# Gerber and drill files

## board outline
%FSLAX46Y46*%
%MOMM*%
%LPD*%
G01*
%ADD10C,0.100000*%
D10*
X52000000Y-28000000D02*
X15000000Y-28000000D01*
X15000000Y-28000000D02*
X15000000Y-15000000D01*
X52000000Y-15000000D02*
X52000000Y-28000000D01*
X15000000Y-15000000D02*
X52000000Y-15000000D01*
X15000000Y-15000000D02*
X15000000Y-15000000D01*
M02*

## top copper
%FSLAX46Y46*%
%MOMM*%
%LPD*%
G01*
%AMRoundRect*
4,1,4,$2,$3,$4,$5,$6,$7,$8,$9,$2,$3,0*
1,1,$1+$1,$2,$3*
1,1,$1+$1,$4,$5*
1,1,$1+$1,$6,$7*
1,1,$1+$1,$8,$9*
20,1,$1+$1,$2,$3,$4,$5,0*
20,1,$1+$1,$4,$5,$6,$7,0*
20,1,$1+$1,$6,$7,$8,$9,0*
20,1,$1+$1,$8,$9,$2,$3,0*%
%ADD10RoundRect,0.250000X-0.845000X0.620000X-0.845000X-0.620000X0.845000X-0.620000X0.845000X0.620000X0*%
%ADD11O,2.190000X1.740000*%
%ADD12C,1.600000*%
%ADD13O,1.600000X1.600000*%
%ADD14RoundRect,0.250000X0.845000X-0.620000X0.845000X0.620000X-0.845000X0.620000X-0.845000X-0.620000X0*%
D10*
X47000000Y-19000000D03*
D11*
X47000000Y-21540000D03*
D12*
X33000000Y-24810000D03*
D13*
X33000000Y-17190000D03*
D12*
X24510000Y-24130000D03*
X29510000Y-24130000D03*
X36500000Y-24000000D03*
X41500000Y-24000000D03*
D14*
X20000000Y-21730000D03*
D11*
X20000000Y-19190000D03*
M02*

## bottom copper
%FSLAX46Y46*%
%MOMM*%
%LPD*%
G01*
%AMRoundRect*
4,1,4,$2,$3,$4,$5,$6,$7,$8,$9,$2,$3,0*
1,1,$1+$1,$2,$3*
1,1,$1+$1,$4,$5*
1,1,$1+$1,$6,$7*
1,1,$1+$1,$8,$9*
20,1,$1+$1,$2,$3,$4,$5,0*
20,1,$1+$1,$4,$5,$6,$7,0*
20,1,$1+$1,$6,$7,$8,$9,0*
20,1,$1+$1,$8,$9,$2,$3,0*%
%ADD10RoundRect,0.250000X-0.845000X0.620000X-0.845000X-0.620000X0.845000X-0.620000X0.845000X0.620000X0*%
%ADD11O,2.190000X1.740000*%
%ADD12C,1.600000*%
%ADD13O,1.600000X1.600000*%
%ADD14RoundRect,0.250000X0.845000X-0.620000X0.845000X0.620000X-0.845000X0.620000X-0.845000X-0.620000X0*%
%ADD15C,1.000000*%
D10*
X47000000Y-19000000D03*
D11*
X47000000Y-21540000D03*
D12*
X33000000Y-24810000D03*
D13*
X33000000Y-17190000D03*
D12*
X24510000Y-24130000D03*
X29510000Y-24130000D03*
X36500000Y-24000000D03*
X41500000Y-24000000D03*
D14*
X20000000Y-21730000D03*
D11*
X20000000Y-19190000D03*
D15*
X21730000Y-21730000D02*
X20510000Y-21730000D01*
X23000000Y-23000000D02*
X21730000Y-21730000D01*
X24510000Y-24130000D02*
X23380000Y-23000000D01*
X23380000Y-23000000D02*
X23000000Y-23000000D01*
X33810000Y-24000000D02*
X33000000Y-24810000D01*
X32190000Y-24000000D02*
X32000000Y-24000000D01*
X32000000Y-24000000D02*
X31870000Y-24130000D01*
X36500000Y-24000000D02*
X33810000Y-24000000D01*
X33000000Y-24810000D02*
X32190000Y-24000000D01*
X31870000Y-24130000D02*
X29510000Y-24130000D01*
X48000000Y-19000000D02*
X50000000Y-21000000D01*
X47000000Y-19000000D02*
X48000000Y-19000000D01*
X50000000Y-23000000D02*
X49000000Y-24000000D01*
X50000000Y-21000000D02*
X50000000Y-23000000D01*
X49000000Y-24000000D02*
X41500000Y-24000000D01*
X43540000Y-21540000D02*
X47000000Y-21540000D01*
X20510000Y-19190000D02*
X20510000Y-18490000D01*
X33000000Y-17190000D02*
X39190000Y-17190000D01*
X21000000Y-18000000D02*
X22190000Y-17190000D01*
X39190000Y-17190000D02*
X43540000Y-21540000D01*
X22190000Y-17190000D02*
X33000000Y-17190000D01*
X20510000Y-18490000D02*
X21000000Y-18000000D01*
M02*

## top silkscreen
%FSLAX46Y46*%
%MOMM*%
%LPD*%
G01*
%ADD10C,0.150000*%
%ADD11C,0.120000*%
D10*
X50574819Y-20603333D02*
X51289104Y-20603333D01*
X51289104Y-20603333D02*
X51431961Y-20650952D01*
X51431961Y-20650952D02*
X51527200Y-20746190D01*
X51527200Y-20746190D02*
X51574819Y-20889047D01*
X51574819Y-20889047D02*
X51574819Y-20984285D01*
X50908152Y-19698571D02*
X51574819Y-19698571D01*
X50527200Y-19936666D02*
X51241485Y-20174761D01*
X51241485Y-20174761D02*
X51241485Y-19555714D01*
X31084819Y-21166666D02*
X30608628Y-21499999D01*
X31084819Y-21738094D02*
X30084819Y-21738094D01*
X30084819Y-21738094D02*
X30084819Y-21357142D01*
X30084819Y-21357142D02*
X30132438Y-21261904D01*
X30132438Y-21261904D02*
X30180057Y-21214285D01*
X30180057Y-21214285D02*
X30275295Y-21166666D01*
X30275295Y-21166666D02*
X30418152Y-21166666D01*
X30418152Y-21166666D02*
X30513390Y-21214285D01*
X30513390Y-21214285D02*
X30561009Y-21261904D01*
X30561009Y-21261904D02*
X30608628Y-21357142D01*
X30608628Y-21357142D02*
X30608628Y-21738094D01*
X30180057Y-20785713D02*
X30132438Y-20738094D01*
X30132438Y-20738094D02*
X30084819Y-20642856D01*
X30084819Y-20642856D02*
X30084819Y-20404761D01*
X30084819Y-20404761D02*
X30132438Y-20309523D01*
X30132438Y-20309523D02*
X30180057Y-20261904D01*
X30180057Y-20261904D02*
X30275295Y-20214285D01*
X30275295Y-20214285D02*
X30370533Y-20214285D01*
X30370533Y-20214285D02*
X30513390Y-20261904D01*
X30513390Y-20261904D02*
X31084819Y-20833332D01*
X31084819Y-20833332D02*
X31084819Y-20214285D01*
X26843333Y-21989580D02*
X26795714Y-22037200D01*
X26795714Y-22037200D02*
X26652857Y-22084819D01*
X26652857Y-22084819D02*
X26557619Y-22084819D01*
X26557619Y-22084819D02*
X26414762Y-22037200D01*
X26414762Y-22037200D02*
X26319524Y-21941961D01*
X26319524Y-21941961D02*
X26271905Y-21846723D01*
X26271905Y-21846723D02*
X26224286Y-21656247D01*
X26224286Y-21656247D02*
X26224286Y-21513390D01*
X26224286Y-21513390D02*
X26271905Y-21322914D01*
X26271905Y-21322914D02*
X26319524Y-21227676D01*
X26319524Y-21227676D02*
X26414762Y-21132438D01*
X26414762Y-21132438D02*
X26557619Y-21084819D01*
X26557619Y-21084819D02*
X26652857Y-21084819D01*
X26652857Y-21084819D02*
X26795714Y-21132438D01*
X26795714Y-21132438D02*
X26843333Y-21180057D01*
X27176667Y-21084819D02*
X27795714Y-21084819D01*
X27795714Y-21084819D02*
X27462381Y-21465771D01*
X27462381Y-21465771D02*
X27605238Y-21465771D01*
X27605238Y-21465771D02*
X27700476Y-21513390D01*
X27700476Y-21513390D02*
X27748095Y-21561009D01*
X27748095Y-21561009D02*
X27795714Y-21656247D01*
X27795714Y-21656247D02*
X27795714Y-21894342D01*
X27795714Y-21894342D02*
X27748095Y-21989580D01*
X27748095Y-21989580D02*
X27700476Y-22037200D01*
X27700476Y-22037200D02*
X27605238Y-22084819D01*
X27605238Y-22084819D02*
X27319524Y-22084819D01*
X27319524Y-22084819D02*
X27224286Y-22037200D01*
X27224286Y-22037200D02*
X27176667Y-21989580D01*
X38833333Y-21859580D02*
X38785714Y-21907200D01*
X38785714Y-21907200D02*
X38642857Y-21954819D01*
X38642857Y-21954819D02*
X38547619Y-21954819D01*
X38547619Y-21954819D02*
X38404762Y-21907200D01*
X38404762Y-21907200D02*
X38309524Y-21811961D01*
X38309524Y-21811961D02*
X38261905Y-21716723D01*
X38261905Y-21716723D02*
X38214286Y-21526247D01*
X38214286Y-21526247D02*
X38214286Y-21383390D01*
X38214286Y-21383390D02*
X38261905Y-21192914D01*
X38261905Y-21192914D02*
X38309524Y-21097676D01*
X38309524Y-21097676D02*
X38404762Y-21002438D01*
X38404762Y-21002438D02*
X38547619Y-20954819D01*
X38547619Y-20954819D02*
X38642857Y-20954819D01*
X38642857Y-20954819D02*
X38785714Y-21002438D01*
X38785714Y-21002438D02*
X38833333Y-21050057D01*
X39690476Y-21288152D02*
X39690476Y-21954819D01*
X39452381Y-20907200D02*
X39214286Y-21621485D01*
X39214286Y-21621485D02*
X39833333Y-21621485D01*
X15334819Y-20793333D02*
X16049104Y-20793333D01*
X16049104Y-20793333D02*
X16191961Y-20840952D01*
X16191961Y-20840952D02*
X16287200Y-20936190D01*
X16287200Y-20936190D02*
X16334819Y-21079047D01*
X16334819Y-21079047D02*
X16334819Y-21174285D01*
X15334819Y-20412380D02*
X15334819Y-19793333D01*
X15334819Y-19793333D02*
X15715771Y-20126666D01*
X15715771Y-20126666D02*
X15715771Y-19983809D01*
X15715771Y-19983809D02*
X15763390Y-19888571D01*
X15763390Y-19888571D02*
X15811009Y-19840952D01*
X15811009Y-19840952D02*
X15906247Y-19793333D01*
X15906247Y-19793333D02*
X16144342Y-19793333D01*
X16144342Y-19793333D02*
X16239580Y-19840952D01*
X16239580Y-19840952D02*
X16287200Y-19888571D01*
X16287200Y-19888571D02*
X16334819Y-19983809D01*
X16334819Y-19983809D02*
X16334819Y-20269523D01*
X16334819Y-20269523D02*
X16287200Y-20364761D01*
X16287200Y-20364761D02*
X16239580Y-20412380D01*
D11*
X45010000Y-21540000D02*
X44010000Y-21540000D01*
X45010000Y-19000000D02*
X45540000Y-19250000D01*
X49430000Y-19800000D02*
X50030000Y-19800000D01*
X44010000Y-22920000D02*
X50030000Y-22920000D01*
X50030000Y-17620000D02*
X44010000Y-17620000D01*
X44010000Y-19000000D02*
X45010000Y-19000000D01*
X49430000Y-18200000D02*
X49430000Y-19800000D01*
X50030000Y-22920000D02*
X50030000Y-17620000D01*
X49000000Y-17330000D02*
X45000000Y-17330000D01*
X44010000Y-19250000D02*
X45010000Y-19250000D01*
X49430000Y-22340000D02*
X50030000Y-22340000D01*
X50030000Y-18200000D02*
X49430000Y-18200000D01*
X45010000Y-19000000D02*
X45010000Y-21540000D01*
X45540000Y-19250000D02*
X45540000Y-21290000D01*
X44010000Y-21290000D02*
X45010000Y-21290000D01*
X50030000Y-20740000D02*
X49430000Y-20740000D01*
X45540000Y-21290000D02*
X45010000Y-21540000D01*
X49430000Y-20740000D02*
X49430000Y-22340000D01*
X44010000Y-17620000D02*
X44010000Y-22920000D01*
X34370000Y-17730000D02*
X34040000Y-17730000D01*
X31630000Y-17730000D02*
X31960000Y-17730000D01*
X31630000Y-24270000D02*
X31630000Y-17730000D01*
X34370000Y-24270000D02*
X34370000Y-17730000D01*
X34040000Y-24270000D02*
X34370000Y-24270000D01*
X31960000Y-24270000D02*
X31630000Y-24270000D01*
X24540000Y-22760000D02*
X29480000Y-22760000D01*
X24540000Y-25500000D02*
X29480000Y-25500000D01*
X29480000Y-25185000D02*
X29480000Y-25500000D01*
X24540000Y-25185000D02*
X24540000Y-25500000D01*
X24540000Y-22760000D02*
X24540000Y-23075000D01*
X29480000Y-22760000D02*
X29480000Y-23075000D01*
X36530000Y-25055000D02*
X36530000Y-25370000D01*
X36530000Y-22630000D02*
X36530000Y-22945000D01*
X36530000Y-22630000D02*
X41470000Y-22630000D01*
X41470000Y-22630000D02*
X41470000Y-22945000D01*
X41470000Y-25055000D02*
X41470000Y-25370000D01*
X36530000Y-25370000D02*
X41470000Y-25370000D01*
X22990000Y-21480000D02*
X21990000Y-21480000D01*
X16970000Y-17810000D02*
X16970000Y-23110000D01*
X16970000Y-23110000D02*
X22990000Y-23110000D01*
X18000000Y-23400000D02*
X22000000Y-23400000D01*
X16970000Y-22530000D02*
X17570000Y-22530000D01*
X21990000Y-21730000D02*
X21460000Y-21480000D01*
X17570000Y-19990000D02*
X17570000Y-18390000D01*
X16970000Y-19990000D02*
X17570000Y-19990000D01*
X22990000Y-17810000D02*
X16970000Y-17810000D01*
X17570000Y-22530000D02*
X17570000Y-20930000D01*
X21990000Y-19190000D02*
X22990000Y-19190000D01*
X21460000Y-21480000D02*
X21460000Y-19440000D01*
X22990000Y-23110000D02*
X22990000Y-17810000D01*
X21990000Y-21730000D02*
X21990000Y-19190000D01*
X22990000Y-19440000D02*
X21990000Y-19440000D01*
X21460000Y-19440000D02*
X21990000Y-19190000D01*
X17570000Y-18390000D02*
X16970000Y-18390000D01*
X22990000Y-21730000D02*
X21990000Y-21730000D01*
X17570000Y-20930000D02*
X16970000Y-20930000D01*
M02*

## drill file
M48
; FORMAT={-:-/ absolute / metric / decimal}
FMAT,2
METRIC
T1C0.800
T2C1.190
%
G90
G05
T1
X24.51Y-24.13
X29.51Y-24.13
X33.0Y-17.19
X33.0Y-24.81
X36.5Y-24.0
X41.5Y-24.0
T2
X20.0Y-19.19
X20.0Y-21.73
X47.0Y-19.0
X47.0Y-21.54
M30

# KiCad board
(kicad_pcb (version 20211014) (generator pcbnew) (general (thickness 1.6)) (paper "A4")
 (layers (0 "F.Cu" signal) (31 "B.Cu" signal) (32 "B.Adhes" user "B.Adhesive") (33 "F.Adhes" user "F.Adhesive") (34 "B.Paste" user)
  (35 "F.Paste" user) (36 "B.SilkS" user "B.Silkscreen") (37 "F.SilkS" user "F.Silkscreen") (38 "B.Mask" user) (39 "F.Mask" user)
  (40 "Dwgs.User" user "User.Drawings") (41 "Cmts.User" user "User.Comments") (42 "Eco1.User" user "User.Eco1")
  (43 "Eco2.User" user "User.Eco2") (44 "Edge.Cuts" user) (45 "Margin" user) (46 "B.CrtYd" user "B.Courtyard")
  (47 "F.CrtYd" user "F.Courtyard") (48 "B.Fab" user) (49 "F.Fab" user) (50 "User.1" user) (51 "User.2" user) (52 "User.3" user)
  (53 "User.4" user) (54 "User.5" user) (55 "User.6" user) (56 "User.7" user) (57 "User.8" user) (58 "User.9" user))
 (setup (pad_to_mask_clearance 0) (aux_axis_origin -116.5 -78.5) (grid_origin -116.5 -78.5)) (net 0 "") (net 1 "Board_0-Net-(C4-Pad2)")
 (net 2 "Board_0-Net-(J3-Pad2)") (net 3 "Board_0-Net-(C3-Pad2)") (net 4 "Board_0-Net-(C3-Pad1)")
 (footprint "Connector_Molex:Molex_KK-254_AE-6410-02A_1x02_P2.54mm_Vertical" (layer "F.Cu") (at 47 19 -90)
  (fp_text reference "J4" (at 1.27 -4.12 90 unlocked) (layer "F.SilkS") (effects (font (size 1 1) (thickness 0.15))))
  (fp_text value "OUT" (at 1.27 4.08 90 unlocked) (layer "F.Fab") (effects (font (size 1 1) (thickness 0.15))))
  (fp_line (start 2.54 1.99) (end 2.54 2.99) (layer "F.SilkS") (width 0.12))
  (fp_line (start 0 1.99) (end 0.25 1.46) (layer "F.SilkS") (width 0.12))
  (fp_line (start 0.8 -2.43) (end 0.8 -3.03) (layer "F.SilkS") (width 0.12))
  (fp_line (start 3.92 2.99) (end 3.92 -3.03) (layer "F.SilkS") (width 0.12))
  (fp_line (start -1.38 -3.03) (end -1.38 2.99) (layer "F.SilkS") (width 0.12))
  (fp_line (start 0 2.99) (end 0 1.99) (layer "F.SilkS") (width 0.12))
  (fp_line (start -0.8 -2.43) (end 0.8 -2.43) (layer "F.SilkS") (width 0.12))
  (fp_line (start 3.92 -3.03) (end -1.38 -3.03) (layer "F.SilkS") (width 0.12))
  (fp_line (start -1.67 -2) (end -1.67 2) (layer "F.SilkS") (width 0.12))
  (fp_line (start 0.25 2.99) (end 0.25 1.99) (layer "F.SilkS") (width 0.12))
  (fp_line (start 3.34 -2.43) (end 3.34 -3.03) (layer "F.SilkS") (width 0.12))
  (fp_line (start -0.8 -3.03) (end -0.8 -2.43) (layer "F.SilkS") (width 0.12))
  (fp_line (start 0 1.99) (end 2.54 1.99) (layer "F.SilkS") (width 0.12))
  (fp_line (start 0.25 1.46) (end 2.29 1.46) (layer "F.SilkS") (width 0.12))
  (fp_line (start 2.29 2.99) (end 2.29 1.99) (layer "F.SilkS") (width 0.12))
  (fp_line (start 1.74 -3.03) (end 1.74 -2.43) (layer "F.SilkS") (width 0.12))
  (fp_line (start 2.29 1.46) (end 2.54 1.99) (layer "F.SilkS") (width 0.12))
  (fp_line (start 1.74 -2.43) (end 3.34 -2.43) (layer "F.SilkS") (width 0.12))
  (fp_line (start -1.38 2.99) (end 3.92 2.99) (layer "F.SilkS") (width 0.12))
  (pad "1" thru_hole roundrect (at 0 0 270) (size 1.74 2.19) (drill 1.19) (layers *.Cu *.Mask) (roundrect_rratio 0.143678)
   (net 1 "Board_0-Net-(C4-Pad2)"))
  (pad "2" thru_hole oval (at 2.54 0 270) (size 1.74 2.19) (drill 1.19) (layers *.Cu *.Mask) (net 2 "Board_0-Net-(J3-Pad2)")))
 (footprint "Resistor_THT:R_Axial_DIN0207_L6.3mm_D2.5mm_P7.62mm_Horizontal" (layer "F.Cu") (at 33 24.81 90)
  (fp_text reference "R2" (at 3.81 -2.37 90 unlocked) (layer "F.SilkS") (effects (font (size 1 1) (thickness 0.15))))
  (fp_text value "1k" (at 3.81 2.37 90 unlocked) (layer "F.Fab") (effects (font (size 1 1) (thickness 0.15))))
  (fp_line (start 7.08 1.37) (end 7.08 1.04) (layer "F.SilkS") (width 0.12))
  (fp_line (start 7.08 -1.37) (end 7.08 -1.04) (layer "F.SilkS") (width 0.12))
  (fp_line (start 0.54 -1.37) (end 7.08 -1.37) (layer "F.SilkS") (width 0.12))
  (fp_line (start 0.54 1.37) (end 7.08 1.37) (layer "F.SilkS") (width 0.12))
  (fp_line (start 0.54 1.04) (end 0.54 1.37) (layer "F.SilkS") (width 0.12))
  (fp_line (start 0.54 -1.04) (end 0.54 -1.37) (layer "F.SilkS") (width 0.12))
  (pad "1" thru_hole circle (at 0 0 90) (size 1.6 1.6) (drill 0.8) (layers *.Cu *.Mask) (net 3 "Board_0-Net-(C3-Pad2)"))
  (pad "2" thru_hole oval (at 7.62 0 90) (size 1.6 1.6) (drill 0.8) (layers *.Cu *.Mask) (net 2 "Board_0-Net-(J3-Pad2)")))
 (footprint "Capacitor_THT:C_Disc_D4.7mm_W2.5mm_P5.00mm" (layer "F.Cu") (at 24.51 24.13)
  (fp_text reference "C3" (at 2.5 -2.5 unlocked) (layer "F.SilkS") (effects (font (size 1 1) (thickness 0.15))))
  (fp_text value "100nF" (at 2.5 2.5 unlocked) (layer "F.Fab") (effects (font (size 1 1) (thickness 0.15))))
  (fp_line (start 0.03 -1.37) (end 4.97 -1.37) (layer "F.SilkS") (width 0.12))
  (fp_line (start 0.03 1.37) (end 4.97 1.37) (layer "F.SilkS") (width 0.12))
  (fp_line (start 4.97 1.055) (end 4.97 1.37) (layer "F.SilkS") (width 0.12))
  (fp_line (start 0.03 1.055) (end 0.03 1.37) (layer "F.SilkS") (width 0.12))
  (fp_line (start 0.03 -1.37) (end 0.03 -1.055) (layer "F.SilkS") (width 0.12))
  (fp_line (start 4.97 -1.37) (end 4.97 -1.055) (layer "F.SilkS") (width 0.12))
  (pad "1" thru_hole circle (at 0 0) (size 1.6 1.6) (drill 0.8) (layers *.Cu *.Mask) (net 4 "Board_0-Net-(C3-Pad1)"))
  (pad "2" thru_hole circle (at 5 0) (size 1.6 1.6) (drill 0.8) (layers *.Cu *.Mask) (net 3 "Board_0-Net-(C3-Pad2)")))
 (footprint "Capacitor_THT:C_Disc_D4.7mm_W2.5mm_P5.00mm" (layer "F.Cu") (at 36.5 24)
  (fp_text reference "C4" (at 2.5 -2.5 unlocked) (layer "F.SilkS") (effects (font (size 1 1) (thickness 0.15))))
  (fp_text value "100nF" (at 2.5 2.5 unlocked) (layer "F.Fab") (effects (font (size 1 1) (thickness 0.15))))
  (fp_line (start 0.03 1.055) (end 0.03 1.37) (layer "F.SilkS") (width 0.12))
  (fp_line (start 0.03 -1.37) (end 0.03 -1.055) (layer "F.SilkS") (width 0.12))
  (fp_line (start 0.03 -1.37) (end 4.97 -1.37) (layer "F.SilkS") (width 0.12))
  (fp_line (start 4.97 -1.37) (end 4.97 -1.055) (layer "F.SilkS") (width 0.12))
  (fp_line (start 4.97 1.055) (end 4.97 1.37) (layer "F.SilkS") (width 0.12))
  (fp_line (start 0.03 1.37) (end 4.97 1.37) (layer "F.SilkS") (width 0.12))
  (pad "1" thru_hole circle (at 0 0) (size 1.6 1.6) (drill 0.8) (layers *.Cu *.Mask) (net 3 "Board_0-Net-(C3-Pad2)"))
  (pad "2" thru_hole circle (at 5 0) (size 1.6 1.6) (drill 0.8) (layers *.Cu *.Mask) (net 1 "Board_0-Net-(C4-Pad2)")))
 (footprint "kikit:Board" (layer "F.Cu") (at 19 15)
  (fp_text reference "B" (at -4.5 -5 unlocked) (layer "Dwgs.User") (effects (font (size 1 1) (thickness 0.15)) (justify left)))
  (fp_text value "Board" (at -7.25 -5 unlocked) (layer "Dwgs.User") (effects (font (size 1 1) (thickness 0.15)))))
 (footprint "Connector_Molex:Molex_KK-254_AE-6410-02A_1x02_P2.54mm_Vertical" (layer "F.Cu") (at 20 21.73 90)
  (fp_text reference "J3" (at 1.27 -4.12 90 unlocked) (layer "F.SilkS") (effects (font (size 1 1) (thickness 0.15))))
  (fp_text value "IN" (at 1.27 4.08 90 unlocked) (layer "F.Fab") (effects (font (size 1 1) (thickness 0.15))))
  (fp_line (start 0.25 2.99) (end 0.25 1.99) (layer "F.SilkS") (width 0.12))
  (fp_line (start 3.92 -3.03) (end -1.38 -3.03) (layer "F.SilkS") (width 0.12))
  (fp_line (start -1.38 -3.03) (end -1.38 2.99) (layer "F.SilkS") (width 0.12))
  (fp_line (start -1.67 -2) (end -1.67 2) (layer "F.SilkS") (width 0.12))
  (fp_line (start -0.8 -3.03) (end -0.8 -2.43) (layer "F.SilkS") (width 0.12))
  (fp_line (start 0 1.99) (end 0.25 1.46) (layer "F.SilkS") (width 0.12))
  (fp_line (start 1.74 -2.43) (end 3.34 -2.43) (layer "F.SilkS") (width 0.12))
  (fp_line (start 1.74 -3.03) (end 1.74 -2.43) (layer "F.SilkS") (width 0.12))
  (fp_line (start 3.92 2.99) (end 3.92 -3.03) (layer "F.SilkS") (width 0.12))
  (fp_line (start -0.8 -2.43) (end 0.8 -2.43) (layer "F.SilkS") (width 0.12))
  (fp_line (start 2.54 1.99) (end 2.54 2.99) (layer "F.SilkS") (width 0.12))
  (fp_line (start 0.25 1.46) (end 2.29 1.46) (layer "F.SilkS") (width 0.12))
  (fp_line (start -1.38 2.99) (end 3.92 2.99) (layer "F.SilkS") (width 0.12))
  (fp_line (start 0 1.99) (end 2.54 1.99) (layer "F.SilkS") (width 0.12))
  (fp_line (start 2.29 2.99) (end 2.29 1.99) (layer "F.SilkS") (width 0.12))
  (fp_line (start 2.29 1.46) (end 2.54 1.99) (layer "F.SilkS") (width 0.12))
  (fp_line (start 3.34 -2.43) (end 3.34 -3.03) (layer "F.SilkS") (width 0.12))
  (fp_line (start 0 2.99) (end 0 1.99) (layer "F.SilkS") (width 0.12))
  (fp_line (start 0.8 -2.43) (end 0.8 -3.03) (layer "F.SilkS") (width 0.12))
  (pad "1" thru_hole roundrect (at 0 0 90) (size 1.74 2.19) (drill 1.19) (layers *.Cu *.Mask) (roundrect_rratio 0.143678)
   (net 4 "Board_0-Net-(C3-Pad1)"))
  (pad "2" thru_hole oval (at 2.54 0 90) (size 1.74 2.19) (drill 1.19) (layers *.Cu *.Mask) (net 2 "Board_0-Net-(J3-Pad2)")))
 (gr_line (start 52 28) (end 15 28) (layer "Edge.Cuts") (width 0.1))
 (gr_line (start 15 28) (end 15 15) (layer "Edge.Cuts") (width 0.1))
 (gr_line (start 52 15) (end 52 28) (layer "Edge.Cuts") (width 0.1))
 (gr_line (start 15 15) (end 52 15) (layer "Edge.Cuts") (width 0.1))
 (gr_line (start 15 15) (end 15 15) (layer "Edge.Cuts") (width 0.1))
 (segment (start 21.73 21.73) (end 20.51 21.73) (width 1) (layer "B.Cu") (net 4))
 (segment (start 23 23) (end 21.73 21.73) (width 1) (layer "B.Cu") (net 4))
 (segment (start 24.51 24.13) (end 23.38 23) (width 1) (layer "B.Cu") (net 4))
 (segment (start 23.38 23) (end 23 23) (width 1) (layer "B.Cu") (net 4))
 (segment (start 33.81 24) (end 33 24.81) (width 1) (layer "B.Cu") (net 3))
 (segment (start 32.19 24) (end 32 24) (width 1) (layer "B.Cu") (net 3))
 (segment (start 32 24) (end 31.87 24.13) (width 1) (layer "B.Cu") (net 3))
 (segment (start 36.5 24) (end 33.81 24) (width 1) (layer "B.Cu") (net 3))
 (segment (start 33 24.81) (end 32.19 24) (width 1) (layer "B.Cu") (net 3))
 (segment (start 31.87 24.13) (end 29.51 24.13) (width 1) (layer "B.Cu") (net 3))
 (segment (start 48 19) (end 50 21) (width 1) (layer "B.Cu") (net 1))
 (segment (start 47 19) (end 48 19) (width 1) (layer "B.Cu") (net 1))
 (segment (start 50 23) (end 49 24) (width 1) (layer "B.Cu") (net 1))
 (segment (start 50 21) (end 50 23) (width 1) (layer "B.Cu") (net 1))
 (segment (start 49 24) (end 41.5 24) (width 1) (layer "B.Cu") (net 1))
 (segment (start 43.54 21.54) (end 47 21.54) (width 1) (layer "B.Cu") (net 2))
 (segment (start 20.51 19.19) (end 20.51 18.49) (width 1) (layer "B.Cu") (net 2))
 (segment (start 33 17.19) (end 39.19 17.19) (width 1) (layer "B.Cu") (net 2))
 (segment (start 21 18) (end 22.19 17.19) (width 1) (layer "B.Cu") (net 2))
 (segment (start 39.19 17.19) (end 43.54 21.54) (width 1) (layer "B.Cu") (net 2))
 (segment (start 22.19 17.19) (end 33 17.19) (width 1) (layer "B.Cu") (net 2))
 (segment (start 20.51 18.49) (end 21 18) (width 1) (layer "B.Cu") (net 2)))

